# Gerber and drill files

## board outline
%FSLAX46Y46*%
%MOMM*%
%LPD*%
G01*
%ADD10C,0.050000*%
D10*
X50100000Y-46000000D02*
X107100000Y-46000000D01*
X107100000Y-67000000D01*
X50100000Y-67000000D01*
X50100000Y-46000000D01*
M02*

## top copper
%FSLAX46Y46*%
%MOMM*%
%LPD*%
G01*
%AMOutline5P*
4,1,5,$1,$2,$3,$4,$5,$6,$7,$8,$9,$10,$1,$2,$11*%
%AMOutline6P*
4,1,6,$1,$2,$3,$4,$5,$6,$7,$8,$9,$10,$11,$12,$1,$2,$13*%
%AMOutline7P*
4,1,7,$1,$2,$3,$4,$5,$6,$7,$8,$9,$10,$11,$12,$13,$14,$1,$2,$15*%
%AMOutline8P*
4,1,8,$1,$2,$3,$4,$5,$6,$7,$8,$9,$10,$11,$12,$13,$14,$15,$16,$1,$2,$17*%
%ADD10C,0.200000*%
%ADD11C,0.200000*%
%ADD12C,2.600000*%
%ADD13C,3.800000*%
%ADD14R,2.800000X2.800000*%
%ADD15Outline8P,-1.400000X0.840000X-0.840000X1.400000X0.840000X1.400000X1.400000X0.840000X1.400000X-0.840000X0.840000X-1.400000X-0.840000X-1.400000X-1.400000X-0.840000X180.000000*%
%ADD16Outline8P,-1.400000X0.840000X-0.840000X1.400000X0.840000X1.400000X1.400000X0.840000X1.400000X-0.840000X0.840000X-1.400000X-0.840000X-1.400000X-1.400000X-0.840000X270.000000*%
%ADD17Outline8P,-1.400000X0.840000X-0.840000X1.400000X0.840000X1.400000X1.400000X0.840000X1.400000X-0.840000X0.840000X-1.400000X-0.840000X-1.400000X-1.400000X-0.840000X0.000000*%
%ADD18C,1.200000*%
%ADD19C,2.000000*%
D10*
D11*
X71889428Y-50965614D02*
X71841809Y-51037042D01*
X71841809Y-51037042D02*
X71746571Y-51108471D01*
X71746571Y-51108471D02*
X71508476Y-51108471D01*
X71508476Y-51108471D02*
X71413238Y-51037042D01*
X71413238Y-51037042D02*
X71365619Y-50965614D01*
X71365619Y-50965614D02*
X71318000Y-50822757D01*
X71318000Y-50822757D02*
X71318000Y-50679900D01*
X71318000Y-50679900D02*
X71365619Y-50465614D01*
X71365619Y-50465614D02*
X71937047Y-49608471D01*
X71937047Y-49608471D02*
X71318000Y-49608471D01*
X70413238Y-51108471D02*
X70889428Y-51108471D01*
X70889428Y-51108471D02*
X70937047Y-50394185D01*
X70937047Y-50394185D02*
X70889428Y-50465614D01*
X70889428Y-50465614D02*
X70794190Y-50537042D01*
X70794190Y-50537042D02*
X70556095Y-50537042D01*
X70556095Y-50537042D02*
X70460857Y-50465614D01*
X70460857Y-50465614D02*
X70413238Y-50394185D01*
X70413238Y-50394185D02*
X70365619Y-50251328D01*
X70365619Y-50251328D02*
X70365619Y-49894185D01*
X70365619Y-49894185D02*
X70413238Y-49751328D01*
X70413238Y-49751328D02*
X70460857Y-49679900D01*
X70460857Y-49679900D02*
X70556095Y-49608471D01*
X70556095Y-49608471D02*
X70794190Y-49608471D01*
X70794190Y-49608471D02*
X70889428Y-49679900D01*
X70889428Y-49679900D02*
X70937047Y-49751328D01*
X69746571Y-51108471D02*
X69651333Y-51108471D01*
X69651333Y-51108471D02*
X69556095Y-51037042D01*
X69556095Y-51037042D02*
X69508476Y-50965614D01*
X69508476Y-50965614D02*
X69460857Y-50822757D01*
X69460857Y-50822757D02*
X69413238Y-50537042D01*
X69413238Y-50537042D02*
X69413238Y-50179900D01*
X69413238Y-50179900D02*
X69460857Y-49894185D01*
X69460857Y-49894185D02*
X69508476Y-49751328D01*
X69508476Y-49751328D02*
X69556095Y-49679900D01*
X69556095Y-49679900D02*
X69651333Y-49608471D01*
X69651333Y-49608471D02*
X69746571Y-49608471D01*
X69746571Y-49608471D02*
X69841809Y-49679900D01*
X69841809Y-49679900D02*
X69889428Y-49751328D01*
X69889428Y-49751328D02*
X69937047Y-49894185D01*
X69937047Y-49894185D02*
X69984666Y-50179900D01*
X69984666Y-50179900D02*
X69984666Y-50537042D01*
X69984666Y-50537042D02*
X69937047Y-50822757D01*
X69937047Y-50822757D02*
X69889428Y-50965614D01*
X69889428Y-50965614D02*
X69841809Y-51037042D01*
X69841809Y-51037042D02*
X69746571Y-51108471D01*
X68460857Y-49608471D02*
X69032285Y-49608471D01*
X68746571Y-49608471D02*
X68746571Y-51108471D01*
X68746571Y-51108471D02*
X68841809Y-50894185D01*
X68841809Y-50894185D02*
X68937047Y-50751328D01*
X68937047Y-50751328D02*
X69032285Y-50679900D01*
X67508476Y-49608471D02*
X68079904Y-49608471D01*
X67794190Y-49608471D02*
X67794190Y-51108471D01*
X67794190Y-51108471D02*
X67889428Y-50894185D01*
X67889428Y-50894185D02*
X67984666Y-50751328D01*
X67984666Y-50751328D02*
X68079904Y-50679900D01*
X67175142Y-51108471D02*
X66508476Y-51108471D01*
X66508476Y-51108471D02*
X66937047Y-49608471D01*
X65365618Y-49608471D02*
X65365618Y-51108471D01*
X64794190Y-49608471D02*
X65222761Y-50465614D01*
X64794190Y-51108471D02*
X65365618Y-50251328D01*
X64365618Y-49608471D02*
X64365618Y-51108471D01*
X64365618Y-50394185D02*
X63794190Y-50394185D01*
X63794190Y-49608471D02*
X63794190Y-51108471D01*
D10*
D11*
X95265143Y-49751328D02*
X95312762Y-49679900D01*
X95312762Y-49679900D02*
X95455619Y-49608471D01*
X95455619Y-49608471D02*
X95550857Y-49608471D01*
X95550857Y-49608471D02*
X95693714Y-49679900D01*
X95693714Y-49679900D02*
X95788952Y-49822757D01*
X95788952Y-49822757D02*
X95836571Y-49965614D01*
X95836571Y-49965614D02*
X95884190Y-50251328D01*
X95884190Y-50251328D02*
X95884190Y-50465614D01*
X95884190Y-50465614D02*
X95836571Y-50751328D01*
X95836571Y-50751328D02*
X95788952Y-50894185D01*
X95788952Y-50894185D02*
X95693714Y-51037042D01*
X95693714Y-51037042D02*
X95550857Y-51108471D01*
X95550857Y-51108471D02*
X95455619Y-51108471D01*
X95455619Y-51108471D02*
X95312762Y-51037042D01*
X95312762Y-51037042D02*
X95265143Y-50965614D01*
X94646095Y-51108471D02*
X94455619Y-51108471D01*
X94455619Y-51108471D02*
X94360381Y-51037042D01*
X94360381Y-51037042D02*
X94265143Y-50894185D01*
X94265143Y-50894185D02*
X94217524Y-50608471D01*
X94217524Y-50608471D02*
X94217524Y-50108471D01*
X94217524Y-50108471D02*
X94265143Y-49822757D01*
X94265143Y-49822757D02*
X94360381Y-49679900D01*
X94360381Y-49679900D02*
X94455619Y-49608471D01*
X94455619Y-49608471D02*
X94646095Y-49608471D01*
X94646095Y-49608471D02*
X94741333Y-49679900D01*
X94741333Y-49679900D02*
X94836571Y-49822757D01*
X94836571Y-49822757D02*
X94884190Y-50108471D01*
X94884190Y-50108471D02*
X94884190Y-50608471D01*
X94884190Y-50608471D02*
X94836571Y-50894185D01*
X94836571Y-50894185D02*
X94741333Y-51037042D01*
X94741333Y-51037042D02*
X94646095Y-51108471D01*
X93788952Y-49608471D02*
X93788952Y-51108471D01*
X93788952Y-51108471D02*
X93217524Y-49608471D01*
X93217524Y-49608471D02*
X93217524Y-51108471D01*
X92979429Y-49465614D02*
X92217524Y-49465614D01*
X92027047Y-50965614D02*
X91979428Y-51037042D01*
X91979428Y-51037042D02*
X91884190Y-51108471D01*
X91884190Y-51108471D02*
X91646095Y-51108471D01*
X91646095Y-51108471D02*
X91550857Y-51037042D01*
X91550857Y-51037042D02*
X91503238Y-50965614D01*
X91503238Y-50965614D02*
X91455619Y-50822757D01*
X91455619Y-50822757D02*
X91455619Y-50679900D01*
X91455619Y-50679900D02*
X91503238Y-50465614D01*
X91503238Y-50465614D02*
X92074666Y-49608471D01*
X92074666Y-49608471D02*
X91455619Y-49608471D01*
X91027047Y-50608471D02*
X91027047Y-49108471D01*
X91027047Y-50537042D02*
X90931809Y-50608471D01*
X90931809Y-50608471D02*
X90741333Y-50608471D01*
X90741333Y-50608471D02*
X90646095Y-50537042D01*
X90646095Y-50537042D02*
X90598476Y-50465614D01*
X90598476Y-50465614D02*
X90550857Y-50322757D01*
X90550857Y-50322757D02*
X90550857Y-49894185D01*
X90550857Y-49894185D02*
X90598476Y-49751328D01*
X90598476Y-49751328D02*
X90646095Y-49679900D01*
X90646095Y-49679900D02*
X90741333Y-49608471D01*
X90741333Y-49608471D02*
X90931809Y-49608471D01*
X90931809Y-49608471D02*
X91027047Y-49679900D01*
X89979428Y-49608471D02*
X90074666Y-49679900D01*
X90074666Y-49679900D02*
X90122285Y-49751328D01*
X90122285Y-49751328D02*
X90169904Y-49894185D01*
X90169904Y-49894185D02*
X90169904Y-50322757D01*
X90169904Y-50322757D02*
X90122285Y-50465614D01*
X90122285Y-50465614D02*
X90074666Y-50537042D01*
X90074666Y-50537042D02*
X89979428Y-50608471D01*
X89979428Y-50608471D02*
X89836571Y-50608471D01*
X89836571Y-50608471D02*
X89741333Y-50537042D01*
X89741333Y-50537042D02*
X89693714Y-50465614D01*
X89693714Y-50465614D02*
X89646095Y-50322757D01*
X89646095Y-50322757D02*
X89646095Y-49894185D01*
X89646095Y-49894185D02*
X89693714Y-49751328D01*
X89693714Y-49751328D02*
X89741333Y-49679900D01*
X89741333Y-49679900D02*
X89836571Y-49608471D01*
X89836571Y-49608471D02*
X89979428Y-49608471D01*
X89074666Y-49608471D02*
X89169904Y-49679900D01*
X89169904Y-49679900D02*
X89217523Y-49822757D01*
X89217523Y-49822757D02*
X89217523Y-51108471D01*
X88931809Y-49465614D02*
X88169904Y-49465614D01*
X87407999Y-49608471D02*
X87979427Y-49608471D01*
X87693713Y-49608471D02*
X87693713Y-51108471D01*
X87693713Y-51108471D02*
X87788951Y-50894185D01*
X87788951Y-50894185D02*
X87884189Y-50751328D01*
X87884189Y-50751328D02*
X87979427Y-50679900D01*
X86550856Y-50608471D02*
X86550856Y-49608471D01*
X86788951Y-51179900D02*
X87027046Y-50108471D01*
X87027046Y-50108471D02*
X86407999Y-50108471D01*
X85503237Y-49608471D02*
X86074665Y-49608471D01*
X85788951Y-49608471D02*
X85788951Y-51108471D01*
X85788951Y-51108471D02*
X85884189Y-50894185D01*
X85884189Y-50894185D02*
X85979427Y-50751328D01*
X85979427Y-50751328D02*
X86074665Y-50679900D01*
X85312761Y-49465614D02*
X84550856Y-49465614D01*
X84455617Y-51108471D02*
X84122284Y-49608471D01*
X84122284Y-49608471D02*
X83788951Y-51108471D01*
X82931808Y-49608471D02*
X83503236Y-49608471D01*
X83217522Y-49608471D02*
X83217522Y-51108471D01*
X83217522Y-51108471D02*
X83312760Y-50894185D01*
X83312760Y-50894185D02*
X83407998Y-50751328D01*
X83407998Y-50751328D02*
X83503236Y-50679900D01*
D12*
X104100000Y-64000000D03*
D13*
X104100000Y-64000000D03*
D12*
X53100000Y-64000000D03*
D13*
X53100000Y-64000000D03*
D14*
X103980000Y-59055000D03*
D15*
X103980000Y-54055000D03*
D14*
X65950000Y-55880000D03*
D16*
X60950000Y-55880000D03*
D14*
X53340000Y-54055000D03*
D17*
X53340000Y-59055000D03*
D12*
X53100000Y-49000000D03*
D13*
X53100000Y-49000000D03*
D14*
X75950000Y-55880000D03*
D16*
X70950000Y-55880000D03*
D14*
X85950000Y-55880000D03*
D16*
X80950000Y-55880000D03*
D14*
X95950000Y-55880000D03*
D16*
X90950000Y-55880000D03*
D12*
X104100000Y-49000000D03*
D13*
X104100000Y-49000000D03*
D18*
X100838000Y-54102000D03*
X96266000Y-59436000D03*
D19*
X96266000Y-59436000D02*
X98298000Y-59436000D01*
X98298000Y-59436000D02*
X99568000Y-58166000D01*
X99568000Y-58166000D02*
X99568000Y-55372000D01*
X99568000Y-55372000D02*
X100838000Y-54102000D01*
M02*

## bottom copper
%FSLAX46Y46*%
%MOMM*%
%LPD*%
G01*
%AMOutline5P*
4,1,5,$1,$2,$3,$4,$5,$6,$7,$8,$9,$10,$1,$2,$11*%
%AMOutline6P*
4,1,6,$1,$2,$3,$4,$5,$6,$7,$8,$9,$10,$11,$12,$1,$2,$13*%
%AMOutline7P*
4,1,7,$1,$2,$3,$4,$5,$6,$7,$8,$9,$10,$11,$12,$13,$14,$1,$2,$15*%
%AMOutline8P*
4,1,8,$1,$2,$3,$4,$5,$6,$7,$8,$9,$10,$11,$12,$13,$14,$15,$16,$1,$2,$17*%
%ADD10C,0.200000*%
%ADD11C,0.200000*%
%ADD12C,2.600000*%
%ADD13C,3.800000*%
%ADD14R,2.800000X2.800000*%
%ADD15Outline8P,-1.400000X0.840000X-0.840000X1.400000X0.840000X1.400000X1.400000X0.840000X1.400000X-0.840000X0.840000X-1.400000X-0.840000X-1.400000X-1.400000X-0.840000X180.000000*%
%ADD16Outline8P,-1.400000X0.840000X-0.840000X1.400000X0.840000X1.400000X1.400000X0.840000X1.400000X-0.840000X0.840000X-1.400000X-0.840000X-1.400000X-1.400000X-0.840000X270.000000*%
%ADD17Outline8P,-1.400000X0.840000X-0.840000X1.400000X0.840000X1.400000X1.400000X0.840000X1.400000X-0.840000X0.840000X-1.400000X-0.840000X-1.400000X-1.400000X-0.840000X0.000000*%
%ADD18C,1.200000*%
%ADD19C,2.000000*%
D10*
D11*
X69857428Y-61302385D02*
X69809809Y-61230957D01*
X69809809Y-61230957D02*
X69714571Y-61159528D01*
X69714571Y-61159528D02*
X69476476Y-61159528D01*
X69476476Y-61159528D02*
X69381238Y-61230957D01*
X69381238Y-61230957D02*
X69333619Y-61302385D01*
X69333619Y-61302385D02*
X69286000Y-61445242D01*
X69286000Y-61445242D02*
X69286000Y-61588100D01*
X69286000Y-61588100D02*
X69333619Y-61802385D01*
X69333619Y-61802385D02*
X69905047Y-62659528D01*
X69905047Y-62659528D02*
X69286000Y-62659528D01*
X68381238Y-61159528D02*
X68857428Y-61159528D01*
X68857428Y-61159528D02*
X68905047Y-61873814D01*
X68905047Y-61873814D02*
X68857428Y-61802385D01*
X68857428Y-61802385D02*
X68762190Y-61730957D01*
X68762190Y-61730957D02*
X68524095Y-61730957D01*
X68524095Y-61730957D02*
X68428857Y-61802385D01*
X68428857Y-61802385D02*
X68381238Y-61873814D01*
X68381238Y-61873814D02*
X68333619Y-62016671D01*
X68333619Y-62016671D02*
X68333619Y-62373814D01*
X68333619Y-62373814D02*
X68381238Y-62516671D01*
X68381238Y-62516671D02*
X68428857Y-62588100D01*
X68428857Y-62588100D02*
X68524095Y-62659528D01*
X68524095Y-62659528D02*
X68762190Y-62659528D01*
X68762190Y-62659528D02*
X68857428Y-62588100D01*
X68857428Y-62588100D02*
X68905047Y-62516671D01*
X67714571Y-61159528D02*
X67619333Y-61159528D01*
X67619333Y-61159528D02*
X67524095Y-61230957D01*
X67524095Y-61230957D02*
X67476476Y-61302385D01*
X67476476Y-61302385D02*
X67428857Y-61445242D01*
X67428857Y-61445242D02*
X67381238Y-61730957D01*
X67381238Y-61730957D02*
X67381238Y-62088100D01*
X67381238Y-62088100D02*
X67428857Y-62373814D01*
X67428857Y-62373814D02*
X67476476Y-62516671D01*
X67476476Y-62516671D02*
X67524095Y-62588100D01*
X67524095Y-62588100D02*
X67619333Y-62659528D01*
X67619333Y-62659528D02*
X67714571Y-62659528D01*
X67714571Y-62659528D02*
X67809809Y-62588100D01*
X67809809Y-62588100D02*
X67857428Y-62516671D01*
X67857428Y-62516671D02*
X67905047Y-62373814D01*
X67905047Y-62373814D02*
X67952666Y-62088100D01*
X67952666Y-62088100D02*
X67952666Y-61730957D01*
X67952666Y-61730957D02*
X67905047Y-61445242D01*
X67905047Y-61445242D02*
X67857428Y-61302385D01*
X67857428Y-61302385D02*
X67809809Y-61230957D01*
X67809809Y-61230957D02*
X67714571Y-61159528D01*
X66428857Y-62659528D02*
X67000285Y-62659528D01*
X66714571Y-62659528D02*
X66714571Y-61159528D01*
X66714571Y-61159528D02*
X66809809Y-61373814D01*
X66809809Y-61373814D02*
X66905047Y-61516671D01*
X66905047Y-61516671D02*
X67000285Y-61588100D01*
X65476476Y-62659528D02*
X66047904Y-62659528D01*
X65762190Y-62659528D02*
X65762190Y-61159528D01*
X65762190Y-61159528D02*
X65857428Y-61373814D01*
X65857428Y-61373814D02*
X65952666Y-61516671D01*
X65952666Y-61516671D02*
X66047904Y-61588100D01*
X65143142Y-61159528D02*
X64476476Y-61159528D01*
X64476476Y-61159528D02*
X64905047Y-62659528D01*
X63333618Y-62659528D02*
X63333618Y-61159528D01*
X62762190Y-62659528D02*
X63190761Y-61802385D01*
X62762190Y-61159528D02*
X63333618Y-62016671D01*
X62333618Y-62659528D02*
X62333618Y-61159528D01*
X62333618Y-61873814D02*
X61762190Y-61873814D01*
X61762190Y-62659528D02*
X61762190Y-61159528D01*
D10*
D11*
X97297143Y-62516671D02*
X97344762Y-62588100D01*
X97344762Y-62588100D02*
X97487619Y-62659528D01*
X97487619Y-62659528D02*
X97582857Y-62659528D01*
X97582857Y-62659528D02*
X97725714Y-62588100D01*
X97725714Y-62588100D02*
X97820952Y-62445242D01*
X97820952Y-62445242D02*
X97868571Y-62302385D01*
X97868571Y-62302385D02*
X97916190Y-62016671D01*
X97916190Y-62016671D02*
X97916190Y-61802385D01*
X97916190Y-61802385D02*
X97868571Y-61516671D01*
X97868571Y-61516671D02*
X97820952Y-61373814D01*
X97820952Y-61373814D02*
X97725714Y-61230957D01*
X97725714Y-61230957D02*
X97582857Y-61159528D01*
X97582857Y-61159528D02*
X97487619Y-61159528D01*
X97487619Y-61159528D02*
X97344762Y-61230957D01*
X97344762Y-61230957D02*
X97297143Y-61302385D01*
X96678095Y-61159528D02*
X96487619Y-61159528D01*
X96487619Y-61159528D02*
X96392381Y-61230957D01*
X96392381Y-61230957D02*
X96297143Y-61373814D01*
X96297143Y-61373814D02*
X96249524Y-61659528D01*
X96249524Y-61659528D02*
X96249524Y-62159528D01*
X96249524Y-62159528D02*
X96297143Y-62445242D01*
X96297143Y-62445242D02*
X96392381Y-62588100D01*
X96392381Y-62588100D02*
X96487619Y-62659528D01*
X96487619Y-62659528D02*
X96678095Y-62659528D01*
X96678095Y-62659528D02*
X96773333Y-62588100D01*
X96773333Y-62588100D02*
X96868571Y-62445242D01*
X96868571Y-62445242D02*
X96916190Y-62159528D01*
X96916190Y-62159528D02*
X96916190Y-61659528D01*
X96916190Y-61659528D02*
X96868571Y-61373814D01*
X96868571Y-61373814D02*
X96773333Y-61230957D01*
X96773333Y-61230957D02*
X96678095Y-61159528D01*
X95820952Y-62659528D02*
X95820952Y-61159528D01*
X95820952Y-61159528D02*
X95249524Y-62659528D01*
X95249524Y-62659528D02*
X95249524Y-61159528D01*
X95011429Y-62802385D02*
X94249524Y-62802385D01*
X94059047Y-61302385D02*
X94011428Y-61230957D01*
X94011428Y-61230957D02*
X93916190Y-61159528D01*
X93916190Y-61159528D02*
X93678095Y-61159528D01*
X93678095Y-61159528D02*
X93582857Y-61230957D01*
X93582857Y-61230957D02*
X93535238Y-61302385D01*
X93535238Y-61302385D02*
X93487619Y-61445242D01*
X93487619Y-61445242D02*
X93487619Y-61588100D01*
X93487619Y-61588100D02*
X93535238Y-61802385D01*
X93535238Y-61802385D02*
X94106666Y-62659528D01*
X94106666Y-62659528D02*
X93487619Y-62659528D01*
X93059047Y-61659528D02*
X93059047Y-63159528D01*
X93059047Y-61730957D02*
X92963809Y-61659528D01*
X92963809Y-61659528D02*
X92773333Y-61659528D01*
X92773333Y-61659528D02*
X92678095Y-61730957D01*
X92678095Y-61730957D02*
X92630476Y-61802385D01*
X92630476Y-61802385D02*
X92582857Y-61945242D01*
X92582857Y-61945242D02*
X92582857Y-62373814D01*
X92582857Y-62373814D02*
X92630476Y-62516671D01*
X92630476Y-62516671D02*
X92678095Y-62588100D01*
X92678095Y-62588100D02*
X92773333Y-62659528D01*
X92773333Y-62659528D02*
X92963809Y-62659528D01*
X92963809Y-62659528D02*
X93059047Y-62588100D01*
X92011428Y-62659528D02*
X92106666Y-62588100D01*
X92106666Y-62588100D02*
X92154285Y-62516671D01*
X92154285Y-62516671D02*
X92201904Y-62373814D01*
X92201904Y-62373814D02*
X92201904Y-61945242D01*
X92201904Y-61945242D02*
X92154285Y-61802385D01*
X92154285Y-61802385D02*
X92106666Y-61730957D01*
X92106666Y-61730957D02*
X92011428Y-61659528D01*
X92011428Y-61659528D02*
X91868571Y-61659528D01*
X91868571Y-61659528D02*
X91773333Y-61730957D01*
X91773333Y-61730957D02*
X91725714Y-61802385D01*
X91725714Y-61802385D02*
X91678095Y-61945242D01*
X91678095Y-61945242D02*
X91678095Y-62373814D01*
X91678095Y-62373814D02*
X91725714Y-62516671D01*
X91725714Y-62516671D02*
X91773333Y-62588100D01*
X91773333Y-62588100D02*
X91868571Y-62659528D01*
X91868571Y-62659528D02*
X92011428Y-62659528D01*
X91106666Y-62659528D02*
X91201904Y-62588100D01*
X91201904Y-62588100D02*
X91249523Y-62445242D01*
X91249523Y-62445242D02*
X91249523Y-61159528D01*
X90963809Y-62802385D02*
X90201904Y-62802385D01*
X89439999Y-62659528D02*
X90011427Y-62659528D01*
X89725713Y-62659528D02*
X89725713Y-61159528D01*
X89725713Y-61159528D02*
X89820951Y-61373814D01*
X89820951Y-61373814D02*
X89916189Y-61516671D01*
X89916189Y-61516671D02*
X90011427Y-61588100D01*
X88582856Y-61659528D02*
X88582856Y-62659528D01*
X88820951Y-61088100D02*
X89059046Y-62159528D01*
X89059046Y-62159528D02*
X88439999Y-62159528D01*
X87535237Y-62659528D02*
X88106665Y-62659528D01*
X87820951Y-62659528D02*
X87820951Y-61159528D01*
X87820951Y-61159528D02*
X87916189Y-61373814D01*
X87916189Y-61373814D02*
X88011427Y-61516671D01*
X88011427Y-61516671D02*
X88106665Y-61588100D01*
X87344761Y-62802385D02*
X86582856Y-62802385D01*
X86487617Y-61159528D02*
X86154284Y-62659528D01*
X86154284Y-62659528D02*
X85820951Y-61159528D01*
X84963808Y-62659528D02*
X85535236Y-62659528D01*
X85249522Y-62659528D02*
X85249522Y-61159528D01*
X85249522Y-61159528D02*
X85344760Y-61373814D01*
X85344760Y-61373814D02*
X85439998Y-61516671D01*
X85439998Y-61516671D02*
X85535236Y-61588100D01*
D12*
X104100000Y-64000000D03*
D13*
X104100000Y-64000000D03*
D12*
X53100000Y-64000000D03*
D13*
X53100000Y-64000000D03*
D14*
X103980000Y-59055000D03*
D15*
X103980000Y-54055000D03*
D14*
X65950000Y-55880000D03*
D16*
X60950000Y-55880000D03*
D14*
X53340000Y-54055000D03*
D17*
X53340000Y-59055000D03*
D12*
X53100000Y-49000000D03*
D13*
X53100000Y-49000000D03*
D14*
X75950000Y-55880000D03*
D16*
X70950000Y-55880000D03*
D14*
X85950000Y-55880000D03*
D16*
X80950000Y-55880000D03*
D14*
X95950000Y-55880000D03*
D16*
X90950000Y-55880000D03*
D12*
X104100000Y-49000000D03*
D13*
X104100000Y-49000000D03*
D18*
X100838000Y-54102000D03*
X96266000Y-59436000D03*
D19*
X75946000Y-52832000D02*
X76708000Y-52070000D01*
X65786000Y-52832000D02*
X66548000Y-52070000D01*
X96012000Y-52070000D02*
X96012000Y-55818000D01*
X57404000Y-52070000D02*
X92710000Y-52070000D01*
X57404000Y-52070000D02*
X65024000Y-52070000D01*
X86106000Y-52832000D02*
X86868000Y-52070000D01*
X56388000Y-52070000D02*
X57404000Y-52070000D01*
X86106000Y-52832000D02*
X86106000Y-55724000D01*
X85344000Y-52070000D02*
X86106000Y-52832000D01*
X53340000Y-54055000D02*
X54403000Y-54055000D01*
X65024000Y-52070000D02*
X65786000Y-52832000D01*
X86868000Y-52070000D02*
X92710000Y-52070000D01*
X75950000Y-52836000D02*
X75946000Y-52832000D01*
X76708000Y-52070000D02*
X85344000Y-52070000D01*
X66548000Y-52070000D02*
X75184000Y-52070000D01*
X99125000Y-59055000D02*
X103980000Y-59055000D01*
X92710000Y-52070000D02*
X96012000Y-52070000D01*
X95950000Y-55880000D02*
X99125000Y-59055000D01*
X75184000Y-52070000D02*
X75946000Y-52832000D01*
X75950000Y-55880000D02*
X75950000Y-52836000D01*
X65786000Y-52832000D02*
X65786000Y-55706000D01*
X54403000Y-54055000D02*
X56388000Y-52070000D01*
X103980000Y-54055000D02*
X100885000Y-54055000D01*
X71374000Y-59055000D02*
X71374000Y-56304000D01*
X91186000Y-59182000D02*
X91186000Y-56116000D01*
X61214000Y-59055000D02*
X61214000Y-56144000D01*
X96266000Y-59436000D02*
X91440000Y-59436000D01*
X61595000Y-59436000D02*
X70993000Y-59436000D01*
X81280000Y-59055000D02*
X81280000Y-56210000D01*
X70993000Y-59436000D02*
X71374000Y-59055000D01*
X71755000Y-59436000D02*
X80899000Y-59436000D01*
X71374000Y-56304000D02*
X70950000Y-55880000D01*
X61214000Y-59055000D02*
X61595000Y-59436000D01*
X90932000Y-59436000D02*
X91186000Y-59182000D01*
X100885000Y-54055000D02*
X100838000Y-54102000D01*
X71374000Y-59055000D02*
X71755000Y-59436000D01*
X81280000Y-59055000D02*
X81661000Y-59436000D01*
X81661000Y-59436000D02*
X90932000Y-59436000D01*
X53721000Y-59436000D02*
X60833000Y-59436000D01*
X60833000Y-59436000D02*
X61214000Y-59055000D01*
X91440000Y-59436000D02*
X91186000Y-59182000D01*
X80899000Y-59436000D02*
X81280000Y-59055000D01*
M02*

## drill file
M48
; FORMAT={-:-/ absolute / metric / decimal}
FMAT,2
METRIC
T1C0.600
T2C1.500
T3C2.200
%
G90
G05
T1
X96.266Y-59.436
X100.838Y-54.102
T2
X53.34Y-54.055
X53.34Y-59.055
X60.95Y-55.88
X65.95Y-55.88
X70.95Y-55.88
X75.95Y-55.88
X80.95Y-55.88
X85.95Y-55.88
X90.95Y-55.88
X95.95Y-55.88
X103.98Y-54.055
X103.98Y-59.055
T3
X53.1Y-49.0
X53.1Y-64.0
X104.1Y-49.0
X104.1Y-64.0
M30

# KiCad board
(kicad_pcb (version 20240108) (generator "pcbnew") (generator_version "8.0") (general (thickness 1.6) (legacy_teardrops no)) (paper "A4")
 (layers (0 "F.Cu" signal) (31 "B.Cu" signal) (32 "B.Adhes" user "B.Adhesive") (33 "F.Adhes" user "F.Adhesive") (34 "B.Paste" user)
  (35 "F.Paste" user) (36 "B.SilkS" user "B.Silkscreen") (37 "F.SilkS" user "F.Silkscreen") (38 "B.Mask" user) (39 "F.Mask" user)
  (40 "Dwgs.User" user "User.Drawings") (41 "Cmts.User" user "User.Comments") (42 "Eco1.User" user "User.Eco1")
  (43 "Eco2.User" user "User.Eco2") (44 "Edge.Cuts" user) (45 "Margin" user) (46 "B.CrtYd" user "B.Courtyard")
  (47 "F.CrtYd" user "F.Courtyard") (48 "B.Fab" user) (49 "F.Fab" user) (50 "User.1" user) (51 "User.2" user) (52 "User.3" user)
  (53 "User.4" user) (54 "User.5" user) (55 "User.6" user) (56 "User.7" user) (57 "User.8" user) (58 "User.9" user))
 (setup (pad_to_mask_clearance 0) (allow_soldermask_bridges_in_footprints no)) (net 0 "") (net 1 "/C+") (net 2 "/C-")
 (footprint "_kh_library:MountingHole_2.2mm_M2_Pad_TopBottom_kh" (layer "F.Cu") (at 104.1 64)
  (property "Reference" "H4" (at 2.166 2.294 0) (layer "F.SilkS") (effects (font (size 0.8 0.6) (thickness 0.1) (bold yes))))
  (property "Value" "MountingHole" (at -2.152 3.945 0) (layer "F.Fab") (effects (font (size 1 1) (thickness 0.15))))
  (pad "1" thru_hole circle (at 0 0) (size 2.6 2.6) (drill 2.2) (layers "*.Cu" "*.Mask") (remove_unused_layers no))
  (pad "1" connect circle (at 0 0) (size 3.8 3.8) (layers "F.Cu" "F.Mask"))
  (pad "1" connect circle (at 0 0) (size 3.8 3.8) (layers "B.Cu" "B.Mask")))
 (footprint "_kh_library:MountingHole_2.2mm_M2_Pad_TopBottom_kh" (layer "F.Cu") (at 53.1 64)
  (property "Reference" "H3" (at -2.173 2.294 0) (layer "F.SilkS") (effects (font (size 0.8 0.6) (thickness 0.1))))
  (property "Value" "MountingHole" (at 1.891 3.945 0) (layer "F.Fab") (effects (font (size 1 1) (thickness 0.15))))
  (pad "1" thru_hole circle (at 0 0) (size 2.6 2.6) (drill 2.2) (layers "*.Cu" "*.Mask") (remove_unused_layers no))
  (pad "1" connect circle (at 0 0) (size 3.8 3.8) (layers "F.Cu" "F.Mask"))
  (pad "1" connect circle (at 0 0) (size 3.8 3.8) (layers "B.Cu" "B.Mask")))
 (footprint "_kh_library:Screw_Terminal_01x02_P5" (layer "F.Cu") (at 103.98 59.055 180)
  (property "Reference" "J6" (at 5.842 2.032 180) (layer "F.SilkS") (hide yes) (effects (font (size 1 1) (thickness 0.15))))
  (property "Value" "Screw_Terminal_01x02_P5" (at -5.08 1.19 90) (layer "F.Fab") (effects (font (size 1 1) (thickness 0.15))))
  (pad "1" thru_hole rect (at 0 0 180) (size 2.8 2.8) (drill 1.5) (layers "*.Cu" "*.Mask") (remove_unused_layers no) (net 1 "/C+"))
  (pad "2" thru_hole roundrect (at 0 5 180) (size 2.8 2.8) (drill 1.5) (layers "*.Cu" "*.Mask") (remove_unused_layers no)
   (roundrect_rratio 0) (chamfer_ratio 0.2) (chamfer top_left top_right bottom_left bottom_right) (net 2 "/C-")))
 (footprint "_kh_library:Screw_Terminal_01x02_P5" (layer "F.Cu") (at 65.95 55.88 -90)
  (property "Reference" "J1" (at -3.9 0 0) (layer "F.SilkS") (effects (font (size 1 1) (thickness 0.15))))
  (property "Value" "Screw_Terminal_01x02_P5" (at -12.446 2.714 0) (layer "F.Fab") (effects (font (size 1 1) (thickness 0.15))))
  (pad "1" thru_hole rect (at 0 0 270) (size 2.8 2.8) (drill 1.5) (layers "*.Cu" "*.Mask") (remove_unused_layers no) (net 1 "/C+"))
  (pad "2" thru_hole roundrect (at 0 5 270) (size 2.8 2.8) (drill 1.5) (layers "*.Cu" "*.Mask") (remove_unused_layers no)
   (roundrect_rratio 0) (chamfer_ratio 0.2) (chamfer top_left top_right bottom_left bottom_right) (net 2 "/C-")))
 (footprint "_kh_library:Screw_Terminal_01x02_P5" (layer "F.Cu") (at 53.34 54.055)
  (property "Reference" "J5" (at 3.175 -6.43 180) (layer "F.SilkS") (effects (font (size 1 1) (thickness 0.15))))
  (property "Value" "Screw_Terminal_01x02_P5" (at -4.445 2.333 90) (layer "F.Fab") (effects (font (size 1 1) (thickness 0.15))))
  (pad "1" thru_hole rect (at 0 0) (size 2.8 2.8) (drill 1.5) (layers "*.Cu" "*.Mask") (remove_unused_layers no) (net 1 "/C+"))
  (pad "2" thru_hole roundrect (at 0 5) (size 2.8 2.8) (drill 1.5) (layers "*.Cu" "*.Mask") (remove_unused_layers no) (roundrect_rratio 0)
   (chamfer_ratio 0.2) (chamfer top_left top_right bottom_left bottom_right) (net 2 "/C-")))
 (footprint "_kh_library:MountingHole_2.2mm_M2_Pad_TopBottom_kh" (layer "F.Cu") (at 53.1 49)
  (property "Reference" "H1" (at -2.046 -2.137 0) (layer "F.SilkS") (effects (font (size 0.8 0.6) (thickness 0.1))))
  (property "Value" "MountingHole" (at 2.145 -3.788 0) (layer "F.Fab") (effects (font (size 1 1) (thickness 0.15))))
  (pad "1" thru_hole circle (at 0 0) (size 2.6 2.6) (drill 2.2) (layers "*.Cu" "*.Mask") (remove_unused_layers no))
  (pad "1" connect circle (at 0 0) (size 3.8 3.8) (layers "F.Cu" "F.Mask"))
  (pad "1" connect circle (at 0 0) (size 3.8 3.8) (layers "B.Cu" "B.Mask")))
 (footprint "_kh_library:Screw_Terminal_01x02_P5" (layer "F.Cu") (at 75.95 55.88 -90)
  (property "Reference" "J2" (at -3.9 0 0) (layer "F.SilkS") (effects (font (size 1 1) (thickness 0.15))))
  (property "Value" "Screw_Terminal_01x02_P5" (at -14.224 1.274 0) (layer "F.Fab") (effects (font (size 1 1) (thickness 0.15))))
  (pad "1" thru_hole rect (at 0 0 270) (size 2.8 2.8) (drill 1.5) (layers "*.Cu" "*.Mask") (remove_unused_layers no) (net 1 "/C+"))
  (pad "2" thru_hole roundrect (at 0 5 270) (size 2.8 2.8) (drill 1.5) (layers "*.Cu" "*.Mask") (remove_unused_layers no)
   (roundrect_rratio 0) (chamfer_ratio 0.2) (chamfer top_left top_right bottom_left bottom_right) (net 2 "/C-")))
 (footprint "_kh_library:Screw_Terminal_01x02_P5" (layer "F.Cu") (at 85.95 55.88 -90)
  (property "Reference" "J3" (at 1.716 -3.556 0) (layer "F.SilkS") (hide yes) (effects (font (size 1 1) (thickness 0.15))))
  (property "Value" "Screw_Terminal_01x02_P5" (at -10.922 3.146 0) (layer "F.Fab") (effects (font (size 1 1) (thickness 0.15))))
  (pad "1" thru_hole rect (at 0 0 270) (size 2.8 2.8) (drill 1.5) (layers "*.Cu" "*.Mask") (remove_unused_layers no) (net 1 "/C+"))
  (pad "2" thru_hole roundrect (at 0 5 270) (size 2.8 2.8) (drill 1.5) (layers "*.Cu" "*.Mask") (remove_unused_layers no)
   (roundrect_rratio 0) (chamfer_ratio 0.2) (chamfer top_left top_right bottom_left bottom_right) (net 2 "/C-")))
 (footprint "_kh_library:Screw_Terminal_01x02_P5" (layer "F.Cu") (at 95.95 55.88 -90)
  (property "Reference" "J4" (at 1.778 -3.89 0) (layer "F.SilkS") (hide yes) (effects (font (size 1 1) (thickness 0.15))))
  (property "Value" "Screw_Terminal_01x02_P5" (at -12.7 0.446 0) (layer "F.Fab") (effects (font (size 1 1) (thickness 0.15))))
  (pad "1" thru_hole rect (at 0 0 270) (size 2.8 2.8) (drill 1.5) (layers "*.Cu" "*.Mask") (remove_unused_layers no) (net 1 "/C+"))
  (pad "2" thru_hole roundrect (at 0 5 270) (size 2.8 2.8) (drill 1.5) (layers "*.Cu" "*.Mask") (remove_unused_layers no)
   (roundrect_rratio 0) (chamfer_ratio 0.2) (chamfer top_left top_right bottom_left bottom_right) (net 2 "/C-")))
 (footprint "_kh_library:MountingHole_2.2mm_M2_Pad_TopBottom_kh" (layer "F.Cu") (at 104.1 49)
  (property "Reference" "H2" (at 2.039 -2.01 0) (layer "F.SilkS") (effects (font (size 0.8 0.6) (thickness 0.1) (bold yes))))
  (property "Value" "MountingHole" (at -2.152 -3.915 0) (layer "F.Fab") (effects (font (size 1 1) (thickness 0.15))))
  (pad "1" thru_hole circle (at 0 0) (size 2.6 2.6) (drill 2.2) (layers "*.Cu" "*.Mask") (remove_unused_layers no))
  (pad "1" connect circle (at 0 0) (size 3.8 3.8) (layers "F.Cu" "F.Mask"))
  (pad "1" connect circle (at 0 0) (size 3.8 3.8) (layers "B.Cu" "B.Mask")))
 (gr_rect (start 50.1 46) (end 107.1 67) (stroke (width 0.05) (type default)) (fill none) (layer "Edge.Cuts"))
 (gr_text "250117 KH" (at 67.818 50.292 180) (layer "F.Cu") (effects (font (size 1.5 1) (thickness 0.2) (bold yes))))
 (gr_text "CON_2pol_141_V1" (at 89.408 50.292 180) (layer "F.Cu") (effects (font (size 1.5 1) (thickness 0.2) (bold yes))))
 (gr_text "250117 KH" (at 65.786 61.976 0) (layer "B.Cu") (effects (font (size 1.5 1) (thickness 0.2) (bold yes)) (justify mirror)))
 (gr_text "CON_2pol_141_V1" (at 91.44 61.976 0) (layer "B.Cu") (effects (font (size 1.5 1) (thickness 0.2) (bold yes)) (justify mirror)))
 (segment (start 75.946 52.832) (end 76.708 52.07) (width 2) (layer "B.Cu") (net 1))
 (segment (start 65.786 52.832) (end 66.548 52.07) (width 2) (layer "B.Cu") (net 1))
 (segment (start 96.012 52.07) (end 96.012 55.818) (width 2) (layer "B.Cu") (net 1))
 (segment (start 57.404 52.07) (end 92.71 52.07) (width 2) (layer "B.Cu") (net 1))
 (segment (start 57.404 52.07) (end 65.024 52.07) (width 2) (layer "B.Cu") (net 1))
 (segment (start 86.106 52.832) (end 86.868 52.07) (width 2) (layer "B.Cu") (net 1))
 (segment (start 56.388 52.07) (end 57.404 52.07) (width 2) (layer "B.Cu") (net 1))
 (segment (start 86.106 52.832) (end 86.106 55.724) (width 2) (layer "B.Cu") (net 1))
 (segment (start 85.344 52.07) (end 86.106 52.832) (width 2) (layer "B.Cu") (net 1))
 (segment (start 53.34 54.055) (end 54.403 54.055) (width 2) (layer "B.Cu") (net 1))
 (segment (start 65.024 52.07) (end 65.786 52.832) (width 2) (layer "B.Cu") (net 1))
 (segment (start 86.868 52.07) (end 92.71 52.07) (width 2) (layer "B.Cu") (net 1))
 (segment (start 75.95 52.836) (end 75.946 52.832) (width 2) (layer "B.Cu") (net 1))
 (segment (start 76.708 52.07) (end 85.344 52.07) (width 2) (layer "B.Cu") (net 1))
 (segment (start 66.548 52.07) (end 75.184 52.07) (width 2) (layer "B.Cu") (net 1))
 (segment (start 99.125 59.055) (end 103.98 59.055) (width 2) (layer "B.Cu") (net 1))
 (segment (start 92.71 52.07) (end 96.012 52.07) (width 2) (layer "B.Cu") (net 1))
 (segment (start 95.95 55.88) (end 99.125 59.055) (width 2) (layer "B.Cu") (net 1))
 (segment (start 75.184 52.07) (end 75.946 52.832) (width 2) (layer "B.Cu") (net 1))
 (segment (start 75.95 55.88) (end 75.95 52.836) (width 2) (layer "B.Cu") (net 1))
 (segment (start 65.786 52.832) (end 65.786 55.706) (width 2) (layer "B.Cu") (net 1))
 (segment (start 54.403 54.055) (end 56.388 52.07) (width 2) (layer "B.Cu") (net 1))
 (segment (start 96.266 59.436) (end 98.298 59.436) (width 2) (layer "F.Cu") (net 2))
 (segment (start 98.298 59.436) (end 99.568 58.166) (width 2) (layer "F.Cu") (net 2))
 (segment (start 99.568 58.166) (end 99.568 55.372) (width 2) (layer "F.Cu") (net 2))
 (segment (start 99.568 55.372) (end 100.838 54.102) (width 2) (layer "F.Cu") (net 2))
 (via (at 100.838 54.102) (size 1.2) (drill 0.6) (layers "F.Cu" "B.Cu") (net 2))
 (via (at 96.266 59.436) (size 1.2) (drill 0.6) (layers "F.Cu" "B.Cu") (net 2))
 (segment (start 103.98 54.055) (end 100.885 54.055) (width 2) (layer "B.Cu") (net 2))
 (segment (start 71.374 59.055) (end 71.374 56.304) (width 2) (layer "B.Cu") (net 2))
 (segment (start 91.186 59.182) (end 91.186 56.116) (width 2) (layer "B.Cu") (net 2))
 (segment (start 61.214 59.055) (end 61.214 56.144) (width 2) (layer "B.Cu") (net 2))
 (segment (start 96.266 59.436) (end 91.44 59.436) (width 2) (layer "B.Cu") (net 2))
 (segment (start 61.595 59.436) (end 70.993 59.436) (width 2) (layer "B.Cu") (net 2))
 (segment (start 81.28 59.055) (end 81.28 56.21) (width 2) (layer "B.Cu") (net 2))
 (segment (start 70.993 59.436) (end 71.374 59.055) (width 2) (layer "B.Cu") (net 2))
 (segment (start 71.755 59.436) (end 80.899 59.436) (width 2) (layer "B.Cu") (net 2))
 (segment (start 71.374 56.304) (end 70.95 55.88) (width 2) (layer "B.Cu") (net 2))
 (segment (start 61.214 59.055) (end 61.595 59.436) (width 2) (layer "B.Cu") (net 2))
 (segment (start 90.932 59.436) (end 91.186 59.182) (width 2) (layer "B.Cu") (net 2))
 (segment (start 100.885 54.055) (end 100.838 54.102) (width 2) (layer "B.Cu") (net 2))
 (segment (start 71.374 59.055) (end 71.755 59.436) (width 2) (layer "B.Cu") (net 2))
 (segment (start 81.28 59.055) (end 81.661 59.436) (width 2) (layer "B.Cu") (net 2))
 (segment (start 81.661 59.436) (end 90.932 59.436) (width 2) (layer "B.Cu") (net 2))
 (segment (start 53.721 59.436) (end 60.833 59.436) (width 2) (layer "B.Cu") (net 2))
 (segment (start 60.833 59.436) (end 61.214 59.055) (width 2) (layer "B.Cu") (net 2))
 (segment (start 91.44 59.436) (end 91.186 59.182) (width 2) (layer "B.Cu") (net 2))
 (segment (start 80.899 59.436) (end 81.28 59.055) (width 2) (layer "B.Cu") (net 2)))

